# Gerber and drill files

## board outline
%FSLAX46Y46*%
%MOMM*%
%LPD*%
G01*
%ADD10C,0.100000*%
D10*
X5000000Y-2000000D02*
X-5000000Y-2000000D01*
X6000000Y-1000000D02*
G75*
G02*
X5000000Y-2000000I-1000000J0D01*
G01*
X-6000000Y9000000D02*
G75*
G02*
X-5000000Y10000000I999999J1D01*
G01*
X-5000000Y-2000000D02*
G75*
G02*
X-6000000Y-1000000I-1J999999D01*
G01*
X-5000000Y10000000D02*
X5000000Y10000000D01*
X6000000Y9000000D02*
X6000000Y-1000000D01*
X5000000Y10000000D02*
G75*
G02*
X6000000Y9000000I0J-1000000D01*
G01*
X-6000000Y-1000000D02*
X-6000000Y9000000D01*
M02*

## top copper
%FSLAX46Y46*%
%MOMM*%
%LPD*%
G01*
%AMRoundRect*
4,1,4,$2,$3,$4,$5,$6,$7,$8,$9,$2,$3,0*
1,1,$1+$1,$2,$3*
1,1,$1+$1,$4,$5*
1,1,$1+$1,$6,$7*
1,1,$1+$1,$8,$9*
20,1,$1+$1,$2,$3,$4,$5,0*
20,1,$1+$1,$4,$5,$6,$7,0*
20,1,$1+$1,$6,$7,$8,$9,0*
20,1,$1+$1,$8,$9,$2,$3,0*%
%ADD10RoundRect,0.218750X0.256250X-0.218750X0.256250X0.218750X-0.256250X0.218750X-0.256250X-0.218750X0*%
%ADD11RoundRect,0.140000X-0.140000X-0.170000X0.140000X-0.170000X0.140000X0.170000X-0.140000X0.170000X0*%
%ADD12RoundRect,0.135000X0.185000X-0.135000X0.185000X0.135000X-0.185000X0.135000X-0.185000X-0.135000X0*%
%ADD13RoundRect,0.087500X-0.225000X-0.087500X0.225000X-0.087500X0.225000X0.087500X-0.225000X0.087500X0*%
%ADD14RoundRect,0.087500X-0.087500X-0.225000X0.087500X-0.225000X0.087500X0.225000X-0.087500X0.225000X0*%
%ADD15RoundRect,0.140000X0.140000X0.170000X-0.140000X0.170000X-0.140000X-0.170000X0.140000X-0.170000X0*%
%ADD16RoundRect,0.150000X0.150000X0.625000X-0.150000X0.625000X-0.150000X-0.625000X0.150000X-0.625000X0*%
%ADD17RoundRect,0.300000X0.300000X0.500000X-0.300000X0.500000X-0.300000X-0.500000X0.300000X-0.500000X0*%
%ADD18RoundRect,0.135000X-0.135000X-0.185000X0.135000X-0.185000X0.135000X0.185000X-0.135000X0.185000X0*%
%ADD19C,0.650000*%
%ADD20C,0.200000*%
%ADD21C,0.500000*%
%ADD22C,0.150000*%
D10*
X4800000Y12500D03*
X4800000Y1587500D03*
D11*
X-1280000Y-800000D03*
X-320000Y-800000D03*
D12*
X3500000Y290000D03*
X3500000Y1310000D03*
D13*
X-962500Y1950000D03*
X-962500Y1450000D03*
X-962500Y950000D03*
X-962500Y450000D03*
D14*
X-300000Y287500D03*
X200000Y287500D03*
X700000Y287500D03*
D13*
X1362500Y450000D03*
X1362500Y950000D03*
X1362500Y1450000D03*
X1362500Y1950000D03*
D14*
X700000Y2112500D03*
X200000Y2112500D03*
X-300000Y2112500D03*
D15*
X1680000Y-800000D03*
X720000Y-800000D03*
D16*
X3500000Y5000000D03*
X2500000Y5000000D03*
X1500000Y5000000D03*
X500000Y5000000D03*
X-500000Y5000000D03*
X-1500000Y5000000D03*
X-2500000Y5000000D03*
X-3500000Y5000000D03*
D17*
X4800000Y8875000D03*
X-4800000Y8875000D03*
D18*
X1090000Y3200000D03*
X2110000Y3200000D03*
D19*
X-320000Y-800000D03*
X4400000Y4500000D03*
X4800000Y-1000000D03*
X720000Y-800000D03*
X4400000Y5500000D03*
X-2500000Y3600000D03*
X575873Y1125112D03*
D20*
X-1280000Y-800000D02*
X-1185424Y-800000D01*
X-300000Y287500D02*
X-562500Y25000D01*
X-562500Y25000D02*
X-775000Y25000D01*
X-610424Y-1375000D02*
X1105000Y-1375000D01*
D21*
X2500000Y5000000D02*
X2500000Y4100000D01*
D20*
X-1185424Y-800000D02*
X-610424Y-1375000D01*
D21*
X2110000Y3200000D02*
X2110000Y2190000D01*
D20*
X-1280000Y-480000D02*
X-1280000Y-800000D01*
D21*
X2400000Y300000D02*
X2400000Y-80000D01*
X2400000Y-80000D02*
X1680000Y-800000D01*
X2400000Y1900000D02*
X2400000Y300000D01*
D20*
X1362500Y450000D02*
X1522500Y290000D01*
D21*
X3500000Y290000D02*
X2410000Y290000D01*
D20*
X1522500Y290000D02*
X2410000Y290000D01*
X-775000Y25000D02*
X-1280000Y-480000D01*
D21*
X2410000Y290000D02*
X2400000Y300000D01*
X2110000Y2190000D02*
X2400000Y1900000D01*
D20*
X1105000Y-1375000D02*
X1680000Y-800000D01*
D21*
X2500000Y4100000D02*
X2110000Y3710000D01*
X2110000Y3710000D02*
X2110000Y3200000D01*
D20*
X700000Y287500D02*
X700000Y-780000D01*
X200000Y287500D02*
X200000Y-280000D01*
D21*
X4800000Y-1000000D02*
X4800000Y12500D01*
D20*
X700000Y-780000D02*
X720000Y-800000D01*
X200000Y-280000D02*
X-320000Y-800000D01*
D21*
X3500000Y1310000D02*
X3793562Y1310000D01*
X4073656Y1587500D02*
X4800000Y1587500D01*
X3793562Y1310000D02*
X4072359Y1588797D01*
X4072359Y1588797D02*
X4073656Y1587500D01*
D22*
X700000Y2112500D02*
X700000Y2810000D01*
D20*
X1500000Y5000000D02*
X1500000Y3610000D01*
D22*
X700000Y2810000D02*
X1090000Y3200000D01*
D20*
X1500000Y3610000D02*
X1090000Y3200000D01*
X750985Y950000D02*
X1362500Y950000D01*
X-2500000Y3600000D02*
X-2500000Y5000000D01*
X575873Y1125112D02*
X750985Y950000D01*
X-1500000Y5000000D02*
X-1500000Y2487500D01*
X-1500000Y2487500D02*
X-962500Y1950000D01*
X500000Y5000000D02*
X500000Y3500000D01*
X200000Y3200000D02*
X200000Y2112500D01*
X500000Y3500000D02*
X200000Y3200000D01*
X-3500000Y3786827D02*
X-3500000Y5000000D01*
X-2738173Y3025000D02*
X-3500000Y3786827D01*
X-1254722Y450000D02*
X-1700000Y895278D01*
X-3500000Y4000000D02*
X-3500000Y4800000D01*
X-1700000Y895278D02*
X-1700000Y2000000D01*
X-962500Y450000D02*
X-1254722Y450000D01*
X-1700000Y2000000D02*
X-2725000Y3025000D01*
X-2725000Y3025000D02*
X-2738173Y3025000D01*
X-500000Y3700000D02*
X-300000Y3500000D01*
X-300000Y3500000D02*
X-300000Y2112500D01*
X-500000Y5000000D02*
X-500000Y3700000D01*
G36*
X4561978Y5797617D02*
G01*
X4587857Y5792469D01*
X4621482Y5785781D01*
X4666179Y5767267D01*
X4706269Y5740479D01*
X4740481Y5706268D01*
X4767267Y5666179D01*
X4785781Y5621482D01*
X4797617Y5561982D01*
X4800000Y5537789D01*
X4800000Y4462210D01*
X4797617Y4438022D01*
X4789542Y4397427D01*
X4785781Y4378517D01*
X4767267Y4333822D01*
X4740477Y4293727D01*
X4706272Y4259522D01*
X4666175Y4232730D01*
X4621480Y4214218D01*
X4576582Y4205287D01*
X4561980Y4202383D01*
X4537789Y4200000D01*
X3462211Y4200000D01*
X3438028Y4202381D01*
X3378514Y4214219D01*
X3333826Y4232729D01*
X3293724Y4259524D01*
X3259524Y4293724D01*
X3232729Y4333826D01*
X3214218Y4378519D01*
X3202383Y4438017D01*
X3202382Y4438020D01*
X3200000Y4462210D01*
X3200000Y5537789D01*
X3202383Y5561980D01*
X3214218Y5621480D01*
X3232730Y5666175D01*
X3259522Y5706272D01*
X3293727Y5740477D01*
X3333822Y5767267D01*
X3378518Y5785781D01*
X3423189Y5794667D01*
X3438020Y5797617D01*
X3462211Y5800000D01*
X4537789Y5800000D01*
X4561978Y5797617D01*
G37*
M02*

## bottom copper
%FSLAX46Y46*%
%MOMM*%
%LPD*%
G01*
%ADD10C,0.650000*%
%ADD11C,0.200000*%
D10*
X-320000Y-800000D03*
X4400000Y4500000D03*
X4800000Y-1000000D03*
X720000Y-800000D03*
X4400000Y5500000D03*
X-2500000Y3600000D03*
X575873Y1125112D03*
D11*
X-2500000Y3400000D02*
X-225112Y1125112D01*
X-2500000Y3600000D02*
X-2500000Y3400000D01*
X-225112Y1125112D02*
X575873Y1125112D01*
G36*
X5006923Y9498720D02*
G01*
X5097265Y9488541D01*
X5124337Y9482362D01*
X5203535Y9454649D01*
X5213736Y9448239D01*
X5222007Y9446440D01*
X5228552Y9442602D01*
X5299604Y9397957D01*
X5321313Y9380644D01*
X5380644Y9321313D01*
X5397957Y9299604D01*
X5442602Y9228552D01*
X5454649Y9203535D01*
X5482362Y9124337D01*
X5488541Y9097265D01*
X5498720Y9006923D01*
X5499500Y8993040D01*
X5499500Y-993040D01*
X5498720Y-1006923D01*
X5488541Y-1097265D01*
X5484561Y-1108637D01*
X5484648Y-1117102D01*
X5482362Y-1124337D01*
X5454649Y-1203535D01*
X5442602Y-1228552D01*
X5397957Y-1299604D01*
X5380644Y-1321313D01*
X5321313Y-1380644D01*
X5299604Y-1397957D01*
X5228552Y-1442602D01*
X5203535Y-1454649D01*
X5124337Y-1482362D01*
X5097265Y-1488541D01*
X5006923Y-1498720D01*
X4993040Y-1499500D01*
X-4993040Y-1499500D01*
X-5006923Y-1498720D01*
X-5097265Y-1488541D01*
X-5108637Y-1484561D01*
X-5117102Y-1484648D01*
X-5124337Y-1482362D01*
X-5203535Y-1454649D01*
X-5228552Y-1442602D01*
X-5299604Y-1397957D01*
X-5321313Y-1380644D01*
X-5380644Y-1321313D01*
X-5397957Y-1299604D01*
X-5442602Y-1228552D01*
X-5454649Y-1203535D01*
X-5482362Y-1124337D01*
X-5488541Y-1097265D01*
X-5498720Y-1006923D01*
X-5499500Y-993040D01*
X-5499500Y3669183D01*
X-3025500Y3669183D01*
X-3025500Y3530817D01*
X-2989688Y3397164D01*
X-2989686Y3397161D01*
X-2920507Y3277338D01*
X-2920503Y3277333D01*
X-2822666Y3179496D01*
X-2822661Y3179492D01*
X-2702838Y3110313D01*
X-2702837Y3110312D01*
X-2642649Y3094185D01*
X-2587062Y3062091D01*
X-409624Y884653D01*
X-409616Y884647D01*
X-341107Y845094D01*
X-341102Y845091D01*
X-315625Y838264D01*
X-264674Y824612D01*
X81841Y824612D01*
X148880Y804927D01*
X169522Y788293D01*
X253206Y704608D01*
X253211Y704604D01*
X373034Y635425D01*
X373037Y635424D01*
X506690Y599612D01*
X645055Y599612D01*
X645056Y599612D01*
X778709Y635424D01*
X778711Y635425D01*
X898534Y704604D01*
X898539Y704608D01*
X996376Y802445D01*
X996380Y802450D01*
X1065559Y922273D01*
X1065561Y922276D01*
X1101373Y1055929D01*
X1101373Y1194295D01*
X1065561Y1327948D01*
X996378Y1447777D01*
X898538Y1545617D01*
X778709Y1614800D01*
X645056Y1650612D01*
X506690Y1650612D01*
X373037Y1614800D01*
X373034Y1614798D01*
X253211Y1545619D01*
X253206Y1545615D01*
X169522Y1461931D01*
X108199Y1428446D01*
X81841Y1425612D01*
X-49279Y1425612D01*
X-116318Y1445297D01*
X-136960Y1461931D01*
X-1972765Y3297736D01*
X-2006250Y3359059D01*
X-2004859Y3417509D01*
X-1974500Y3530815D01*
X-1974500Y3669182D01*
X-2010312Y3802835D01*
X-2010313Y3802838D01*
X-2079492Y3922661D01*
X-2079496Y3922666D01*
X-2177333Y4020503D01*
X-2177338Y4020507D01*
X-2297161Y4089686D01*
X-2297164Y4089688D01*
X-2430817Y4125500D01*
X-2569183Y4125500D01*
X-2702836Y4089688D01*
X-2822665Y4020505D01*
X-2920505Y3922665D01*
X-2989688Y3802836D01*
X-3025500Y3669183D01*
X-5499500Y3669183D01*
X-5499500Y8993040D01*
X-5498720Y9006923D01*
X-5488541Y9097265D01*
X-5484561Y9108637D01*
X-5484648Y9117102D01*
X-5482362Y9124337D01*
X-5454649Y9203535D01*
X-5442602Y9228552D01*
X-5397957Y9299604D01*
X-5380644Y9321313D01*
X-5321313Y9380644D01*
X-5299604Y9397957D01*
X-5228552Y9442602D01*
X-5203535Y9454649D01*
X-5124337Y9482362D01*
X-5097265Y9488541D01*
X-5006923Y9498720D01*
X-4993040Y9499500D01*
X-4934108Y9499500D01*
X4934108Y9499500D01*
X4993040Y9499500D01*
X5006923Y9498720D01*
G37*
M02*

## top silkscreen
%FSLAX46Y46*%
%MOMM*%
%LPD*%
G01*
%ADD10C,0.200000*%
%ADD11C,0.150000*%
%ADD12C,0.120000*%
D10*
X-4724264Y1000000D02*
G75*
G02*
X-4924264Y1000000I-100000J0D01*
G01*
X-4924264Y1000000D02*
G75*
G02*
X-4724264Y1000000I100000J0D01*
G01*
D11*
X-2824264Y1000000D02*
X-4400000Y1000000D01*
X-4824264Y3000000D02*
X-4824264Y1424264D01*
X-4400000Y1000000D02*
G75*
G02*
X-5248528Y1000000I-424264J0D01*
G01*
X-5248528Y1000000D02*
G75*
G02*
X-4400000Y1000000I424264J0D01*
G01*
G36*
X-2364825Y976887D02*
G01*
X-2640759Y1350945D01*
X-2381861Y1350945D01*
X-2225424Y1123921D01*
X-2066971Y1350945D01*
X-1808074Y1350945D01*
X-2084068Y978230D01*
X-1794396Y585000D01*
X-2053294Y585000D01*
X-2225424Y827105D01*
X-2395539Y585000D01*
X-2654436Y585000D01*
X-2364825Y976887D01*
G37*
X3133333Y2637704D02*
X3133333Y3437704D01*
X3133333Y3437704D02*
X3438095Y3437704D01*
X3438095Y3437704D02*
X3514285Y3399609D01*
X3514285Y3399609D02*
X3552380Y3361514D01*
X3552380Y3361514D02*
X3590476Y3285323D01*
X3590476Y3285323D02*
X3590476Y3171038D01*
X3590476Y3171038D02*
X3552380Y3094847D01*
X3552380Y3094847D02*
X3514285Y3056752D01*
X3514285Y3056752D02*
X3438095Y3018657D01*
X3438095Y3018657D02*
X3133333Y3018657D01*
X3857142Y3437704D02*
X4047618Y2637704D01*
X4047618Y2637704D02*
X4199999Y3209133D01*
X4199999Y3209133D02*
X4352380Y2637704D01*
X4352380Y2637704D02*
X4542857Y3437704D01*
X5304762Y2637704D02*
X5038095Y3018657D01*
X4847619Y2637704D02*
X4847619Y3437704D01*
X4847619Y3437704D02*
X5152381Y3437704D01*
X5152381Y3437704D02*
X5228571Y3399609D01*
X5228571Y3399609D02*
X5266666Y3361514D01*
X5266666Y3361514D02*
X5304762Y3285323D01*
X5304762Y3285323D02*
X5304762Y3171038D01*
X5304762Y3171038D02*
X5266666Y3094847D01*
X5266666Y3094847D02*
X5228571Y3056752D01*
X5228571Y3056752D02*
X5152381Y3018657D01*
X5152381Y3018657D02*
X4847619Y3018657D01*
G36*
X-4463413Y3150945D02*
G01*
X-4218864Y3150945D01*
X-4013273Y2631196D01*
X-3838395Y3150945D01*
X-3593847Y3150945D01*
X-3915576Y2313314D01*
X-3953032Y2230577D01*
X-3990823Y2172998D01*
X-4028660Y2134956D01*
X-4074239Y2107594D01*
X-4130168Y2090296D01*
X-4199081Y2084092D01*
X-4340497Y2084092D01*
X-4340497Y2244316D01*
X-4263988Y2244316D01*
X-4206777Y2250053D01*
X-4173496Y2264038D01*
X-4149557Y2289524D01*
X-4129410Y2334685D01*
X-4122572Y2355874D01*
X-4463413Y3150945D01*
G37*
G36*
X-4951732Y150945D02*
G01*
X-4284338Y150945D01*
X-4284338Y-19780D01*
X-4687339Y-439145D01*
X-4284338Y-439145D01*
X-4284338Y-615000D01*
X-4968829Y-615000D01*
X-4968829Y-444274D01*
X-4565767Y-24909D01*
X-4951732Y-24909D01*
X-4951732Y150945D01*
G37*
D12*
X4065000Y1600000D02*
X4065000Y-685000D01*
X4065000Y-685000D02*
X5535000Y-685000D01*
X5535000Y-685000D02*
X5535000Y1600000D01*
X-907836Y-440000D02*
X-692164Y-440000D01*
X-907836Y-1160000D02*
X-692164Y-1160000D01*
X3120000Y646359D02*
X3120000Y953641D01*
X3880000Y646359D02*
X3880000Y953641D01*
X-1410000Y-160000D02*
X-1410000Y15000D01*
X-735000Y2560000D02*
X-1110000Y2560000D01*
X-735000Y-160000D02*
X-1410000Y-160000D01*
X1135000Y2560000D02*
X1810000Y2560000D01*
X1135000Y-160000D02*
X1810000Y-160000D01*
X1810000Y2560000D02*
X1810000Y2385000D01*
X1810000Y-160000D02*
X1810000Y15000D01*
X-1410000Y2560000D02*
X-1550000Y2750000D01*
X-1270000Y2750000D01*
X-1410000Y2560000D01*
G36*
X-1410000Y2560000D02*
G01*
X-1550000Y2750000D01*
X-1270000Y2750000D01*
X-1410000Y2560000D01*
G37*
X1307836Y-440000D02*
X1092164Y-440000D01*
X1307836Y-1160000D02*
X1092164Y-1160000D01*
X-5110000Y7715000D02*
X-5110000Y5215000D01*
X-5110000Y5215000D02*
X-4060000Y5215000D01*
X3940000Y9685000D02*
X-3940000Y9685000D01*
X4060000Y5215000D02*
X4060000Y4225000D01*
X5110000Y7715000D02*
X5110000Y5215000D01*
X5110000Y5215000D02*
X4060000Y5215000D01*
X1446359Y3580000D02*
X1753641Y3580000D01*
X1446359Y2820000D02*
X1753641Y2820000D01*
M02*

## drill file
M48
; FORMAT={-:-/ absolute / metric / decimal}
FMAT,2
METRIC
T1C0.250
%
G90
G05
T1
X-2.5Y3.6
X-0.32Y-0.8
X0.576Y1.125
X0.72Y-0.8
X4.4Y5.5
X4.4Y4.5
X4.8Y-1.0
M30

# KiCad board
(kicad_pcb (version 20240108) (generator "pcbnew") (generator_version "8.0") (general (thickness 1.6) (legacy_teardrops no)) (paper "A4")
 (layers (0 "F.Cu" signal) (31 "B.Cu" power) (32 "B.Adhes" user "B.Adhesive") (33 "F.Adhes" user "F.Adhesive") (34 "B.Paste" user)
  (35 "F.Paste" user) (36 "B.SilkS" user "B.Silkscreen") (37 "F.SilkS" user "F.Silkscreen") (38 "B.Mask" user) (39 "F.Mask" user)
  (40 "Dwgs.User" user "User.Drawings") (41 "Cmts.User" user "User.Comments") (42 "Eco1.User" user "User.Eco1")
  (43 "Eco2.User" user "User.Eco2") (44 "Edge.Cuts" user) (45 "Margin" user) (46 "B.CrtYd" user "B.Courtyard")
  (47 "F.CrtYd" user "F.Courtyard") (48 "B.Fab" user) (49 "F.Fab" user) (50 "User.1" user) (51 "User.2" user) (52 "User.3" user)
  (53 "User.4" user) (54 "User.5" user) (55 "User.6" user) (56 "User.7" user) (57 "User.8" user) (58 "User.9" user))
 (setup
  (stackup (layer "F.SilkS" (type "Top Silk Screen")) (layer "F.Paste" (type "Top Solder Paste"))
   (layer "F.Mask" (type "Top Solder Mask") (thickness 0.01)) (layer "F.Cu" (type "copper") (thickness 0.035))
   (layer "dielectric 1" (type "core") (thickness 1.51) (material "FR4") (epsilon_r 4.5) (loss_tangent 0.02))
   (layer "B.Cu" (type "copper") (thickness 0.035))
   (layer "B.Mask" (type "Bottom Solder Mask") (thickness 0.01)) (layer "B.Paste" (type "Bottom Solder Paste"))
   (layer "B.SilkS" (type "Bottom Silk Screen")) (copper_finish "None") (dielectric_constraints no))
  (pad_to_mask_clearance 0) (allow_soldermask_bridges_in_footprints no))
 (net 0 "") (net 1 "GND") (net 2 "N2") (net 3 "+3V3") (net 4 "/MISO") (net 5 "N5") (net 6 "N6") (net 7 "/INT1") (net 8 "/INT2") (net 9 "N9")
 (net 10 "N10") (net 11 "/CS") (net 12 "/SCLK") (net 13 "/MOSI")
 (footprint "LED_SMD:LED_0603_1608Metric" (layer "F.Cu") (at 4.8 -0.8 90)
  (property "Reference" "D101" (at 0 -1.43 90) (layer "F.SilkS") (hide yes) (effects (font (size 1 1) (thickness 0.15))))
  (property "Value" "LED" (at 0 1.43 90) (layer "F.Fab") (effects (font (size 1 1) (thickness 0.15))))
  (fp_line (start 0.8 -0.735) (end -1.485 -0.735) (stroke (width 0.12) (type solid)) (layer "F.SilkS"))
  (fp_line (start -1.485 -0.735) (end -1.485 0.735) (stroke (width 0.12) (type solid)) (layer "F.SilkS"))
  (fp_line (start -1.485 0.735) (end 0.8 0.735) (stroke (width 0.12) (type solid)) (layer "F.SilkS"))
  (pad "1" smd roundrect (at -0.7875 0 90) (size 0.875 0.95) (layers "F.Cu" "F.Paste" "F.Mask") (roundrect_rratio 0.25) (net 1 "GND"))
  (pad "2" smd roundrect (at 0.7875 0 90) (size 0.875 0.95) (layers "F.Cu" "F.Paste" "F.Mask") (roundrect_rratio 0.25) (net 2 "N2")))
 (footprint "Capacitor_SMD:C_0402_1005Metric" (layer "F.Cu") (at -0.8 0.8)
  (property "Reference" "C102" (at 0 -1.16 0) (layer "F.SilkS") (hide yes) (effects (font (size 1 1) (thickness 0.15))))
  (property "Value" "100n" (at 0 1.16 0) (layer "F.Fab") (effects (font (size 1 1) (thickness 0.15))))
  (fp_line (start -0.107836 -0.36) (end 0.107836 -0.36) (stroke (width 0.12) (type solid)) (layer "F.SilkS"))
  (fp_line (start -0.107836 0.36) (end 0.107836 0.36) (stroke (width 0.12) (type solid)) (layer "F.SilkS"))
  (pad "1" smd roundrect (at -0.48 0) (size 0.56 0.62) (layers "F.Cu" "F.Paste" "F.Mask") (roundrect_rratio 0.25) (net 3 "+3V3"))
  (pad "2" smd roundrect (at 0.48 0) (size 0.56 0.62) (layers "F.Cu" "F.Paste" "F.Mask") (roundrect_rratio 0.25) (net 1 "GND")))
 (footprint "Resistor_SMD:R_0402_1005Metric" (layer "F.Cu") (at 3.5 -0.8 90)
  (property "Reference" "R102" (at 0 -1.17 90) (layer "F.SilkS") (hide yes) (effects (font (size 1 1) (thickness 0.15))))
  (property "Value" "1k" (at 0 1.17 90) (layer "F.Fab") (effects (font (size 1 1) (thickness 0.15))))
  (fp_line (start -0.153641 -0.38) (end 0.153641 -0.38) (stroke (width 0.12) (type solid)) (layer "F.SilkS"))
  (fp_line (start -0.153641 0.38) (end 0.153641 0.38) (stroke (width 0.12) (type solid)) (layer "F.SilkS"))
  (pad "1" smd roundrect (at -0.51 0 90) (size 0.54 0.64) (layers "F.Cu" "F.Paste" "F.Mask") (roundrect_rratio 0.25) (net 3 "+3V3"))
  (pad "2" smd roundrect (at 0.51 0 90) (size 0.54 0.64) (layers "F.Cu" "F.Paste" "F.Mask") (roundrect_rratio 0.25) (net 2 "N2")))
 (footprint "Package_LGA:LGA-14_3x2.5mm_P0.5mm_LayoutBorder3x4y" (layer "F.Cu") (at 0.2 -1.2)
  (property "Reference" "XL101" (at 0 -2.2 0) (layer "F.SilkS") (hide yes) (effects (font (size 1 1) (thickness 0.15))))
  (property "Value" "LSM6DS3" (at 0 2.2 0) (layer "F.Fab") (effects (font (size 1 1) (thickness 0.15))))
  (fp_line (start -1.61 1.36) (end -1.61 1.185) (stroke (width 0.12) (type solid)) (layer "F.SilkS"))
  (fp_line (start -0.935 -1.36) (end -1.31 -1.36) (stroke (width 0.12) (type solid)) (layer "F.SilkS"))
  (fp_line (start -0.935 1.36) (end -1.61 1.36) (stroke (width 0.12) (type solid)) (layer "F.SilkS"))
  (fp_line (start 0.935 -1.36) (end 1.61 -1.36) (stroke (width 0.12) (type solid)) (layer "F.SilkS"))
  (fp_line (start 0.935 1.36) (end 1.61 1.36) (stroke (width 0.12) (type solid)) (layer "F.SilkS"))
  (fp_line (start 1.61 -1.36) (end 1.61 -1.185) (stroke (width 0.12) (type solid)) (layer "F.SilkS"))
  (fp_line (start 1.61 1.36) (end 1.61 1.185) (stroke (width 0.12) (type solid)) (layer "F.SilkS"))
  (fp_poly
   (pts (xy -1.61 -1.36) (xy -1.75 -1.55) (xy -1.47 -1.55) (xy -1.61 -1.36)) (stroke (width 0.12) (type solid)) (fill solid)
   (layer "F.SilkS"))
  (pad "1" smd roundrect (at -1.1625 -0.75) (size 0.625 0.35) (layers "F.Cu" "F.Paste" "F.Mask") (roundrect_rratio 0.25) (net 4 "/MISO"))
  (pad "2" smd roundrect (at -1.1625 -0.25) (size 0.625 0.35) (layers "F.Cu" "F.Paste" "F.Mask") (roundrect_rratio 0.25) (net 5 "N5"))
  (pad "3" smd roundrect (at -1.1625 0.25) (size 0.625 0.35) (layers "F.Cu" "F.Paste" "F.Mask") (roundrect_rratio 0.25) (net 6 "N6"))
  (pad "4" smd roundrect (at -1.1625 0.75) (size 0.625 0.35) (layers "F.Cu" "F.Paste" "F.Mask") (roundrect_rratio 0.25) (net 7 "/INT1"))
  (pad "5" smd roundrect (at -0.5 0.9125) (size 0.35 0.625) (layers "F.Cu" "F.Paste" "F.Mask") (roundrect_rratio 0.25) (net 3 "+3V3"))
  (pad "6" smd roundrect (at 0 0.9125) (size 0.35 0.625) (layers "F.Cu" "F.Paste" "F.Mask") (roundrect_rratio 0.25) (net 1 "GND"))
  (pad "7" smd roundrect (at 0.5 0.9125) (size 0.35 0.625) (layers "F.Cu" "F.Paste" "F.Mask") (roundrect_rratio 0.25) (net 1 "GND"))
  (pad "8" smd roundrect (at 1.1625 0.75) (size 0.625 0.35) (layers "F.Cu" "F.Paste" "F.Mask") (roundrect_rratio 0.25) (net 3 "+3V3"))
  (pad "9" smd roundrect (at 1.1625 0.25) (size 0.625 0.35) (layers "F.Cu" "F.Paste" "F.Mask") (roundrect_rratio 0.25) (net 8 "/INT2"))
  (pad "10" smd roundrect (at 1.1625 -0.25) (size 0.625 0.35) (layers "F.Cu" "F.Paste" "F.Mask") (roundrect_rratio 0.25) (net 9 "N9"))
  (pad "11" smd roundrect (at 1.1625 -0.75) (size 0.625 0.35) (layers "F.Cu" "F.Paste" "F.Mask") (roundrect_rratio 0.25) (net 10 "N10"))
  (pad "12" smd roundrect (at 0.5 -0.9125) (size 0.35 0.625) (layers "F.Cu" "F.Paste" "F.Mask") (roundrect_rratio 0.25) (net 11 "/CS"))
  (pad "13" smd roundrect (at 0 -0.9125) (size 0.35 0.625) (layers "F.Cu" "F.Paste" "F.Mask") (roundrect_rratio 0.25) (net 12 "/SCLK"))
  (pad "14" smd roundrect (at -0.5 -0.9125) (size 0.35 0.625) (layers "F.Cu" "F.Paste" "F.Mask") (roundrect_rratio 0.25) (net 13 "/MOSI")))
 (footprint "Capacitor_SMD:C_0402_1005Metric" (layer "F.Cu") (at 1.2 0.8 180)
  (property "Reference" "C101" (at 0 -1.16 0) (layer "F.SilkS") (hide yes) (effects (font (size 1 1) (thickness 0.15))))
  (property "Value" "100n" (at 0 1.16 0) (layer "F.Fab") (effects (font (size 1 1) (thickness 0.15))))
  (fp_line (start -0.107836 0.36) (end 0.107836 0.36) (stroke (width 0.12) (type solid)) (layer "F.SilkS"))
  (fp_line (start -0.107836 -0.36) (end 0.107836 -0.36) (stroke (width 0.12) (type solid)) (layer "F.SilkS"))
  (pad "1" smd roundrect (at -0.48 0 180) (size 0.56 0.62) (layers "F.Cu" "F.Paste" "F.Mask") (roundrect_rratio 0.25) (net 3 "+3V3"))
  (pad "2" smd roundrect (at 0.48 0 180) (size 0.56 0.62) (layers "F.Cu" "F.Paste" "F.Mask") (roundrect_rratio 0.25) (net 1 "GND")))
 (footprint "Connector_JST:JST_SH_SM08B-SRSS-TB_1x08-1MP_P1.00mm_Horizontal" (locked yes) (layer "F.Cu") (at 0 -7 180)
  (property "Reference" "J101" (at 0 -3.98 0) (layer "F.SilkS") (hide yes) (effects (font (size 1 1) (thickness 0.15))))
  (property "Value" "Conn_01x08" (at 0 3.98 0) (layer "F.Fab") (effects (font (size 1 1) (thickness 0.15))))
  (fp_line (start 5.11 0.715) (end 5.11 -1.785) (stroke (width 0.12) (type solid)) (layer "F.SilkS"))
  (fp_line (start 5.11 -1.785) (end 4.06 -1.785) (stroke (width 0.12) (type solid)) (layer "F.SilkS"))
  (fp_line (start -3.94 2.685) (end 3.94 2.685) (stroke (width 0.12) (type solid)) (layer "F.SilkS"))
  (fp_line (start -4.06 -1.785) (end -4.06 -2.775) (stroke (width 0.12) (type solid)) (layer "F.SilkS"))
  (fp_line (start -5.11 0.715) (end -5.11 -1.785) (stroke (width 0.12) (type solid)) (layer "F.SilkS"))
  (fp_line (start -5.11 -1.785) (end -4.06 -1.785) (stroke (width 0.12) (type solid)) (layer "F.SilkS"))
  (pad "1" smd roundrect (at -3.5 -2 180) (size 0.6 1.55) (layers "F.Cu" "F.Paste" "F.Mask") (roundrect_rratio 0.25) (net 1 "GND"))
  (pad "2" smd roundrect (at -2.5 -2 180) (size 0.6 1.55) (layers "F.Cu" "F.Paste" "F.Mask") (roundrect_rratio 0.25) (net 3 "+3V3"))
  (pad "3" smd roundrect (at -1.5 -2 180) (size 0.6 1.55) (layers "F.Cu" "F.Paste" "F.Mask") (roundrect_rratio 0.25) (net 11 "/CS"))
  (pad "4" smd roundrect (at -0.5 -2 180) (size 0.6 1.55) (layers "F.Cu" "F.Paste" "F.Mask") (roundrect_rratio 0.25) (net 12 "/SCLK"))
  (pad "5" smd roundrect (at 0.5 -2 180) (size 0.6 1.55) (layers "F.Cu" "F.Paste" "F.Mask") (roundrect_rratio 0.25) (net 13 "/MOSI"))
  (pad "6" smd roundrect (at 1.5 -2 180) (size 0.6 1.55) (layers "F.Cu" "F.Paste" "F.Mask") (roundrect_rratio 0.25) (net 4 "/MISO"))
  (pad "7" smd roundrect (at 2.5 -2 180) (size 0.6 1.55) (layers "F.Cu" "F.Paste" "F.Mask") (roundrect_rratio 0.25) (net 8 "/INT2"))
  (pad "8" smd roundrect (at 3.5 -2 180) (size 0.6 1.55) (layers "F.Cu" "F.Paste" "F.Mask") (roundrect_rratio 0.25) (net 7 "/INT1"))
  (pad "MP" smd roundrect (at -4.8 1.875 180) (size 1.2 1.6) (layers "F.Cu" "F.Paste" "F.Mask") (roundrect_rratio 0.25))
  (pad "MP" smd roundrect (at 4.8 1.875 180) (size 1.2 1.6) (layers "F.Cu" "F.Paste" "F.Mask") (roundrect_rratio 0.25)))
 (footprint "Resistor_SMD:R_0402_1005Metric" (layer "F.Cu") (at 1.6 -3.2)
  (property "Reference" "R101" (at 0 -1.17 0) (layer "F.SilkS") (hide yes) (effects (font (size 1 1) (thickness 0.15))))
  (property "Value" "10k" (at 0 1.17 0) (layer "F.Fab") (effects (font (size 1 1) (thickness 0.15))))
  (fp_line (start -0.153641 -0.38) (end 0.153641 -0.38) (stroke (width 0.12) (type solid)) (layer "F.SilkS"))
  (fp_line (start -0.153641 0.38) (end 0.153641 0.38) (stroke (width 0.12) (type solid)) (layer "F.SilkS"))
  (pad "1" smd roundrect (at -0.51 0) (size 0.54 0.64) (layers "F.Cu" "F.Paste" "F.Mask") (roundrect_rratio 0.25) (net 11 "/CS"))
  (pad "2" smd roundrect (at 0.51 0) (size 0.54 0.64) (layers "F.Cu" "F.Paste" "F.Mask") (roundrect_rratio 0.25) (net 3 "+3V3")))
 (gr_circle (center -4.824264 -1) (end -4.824264 -0.9) (stroke (width 0.2) (type default)) (fill none) (layer "F.SilkS"))
 (gr_line (start -2.824264 -1) (end -4.4 -1) (stroke (width 0.15) (type default)) (layer "F.SilkS"))
 (gr_line (start -4.824264 -3) (end -4.824264 -1.424264) (stroke (width 0.15) (type default)) (layer "F.SilkS"))
 (gr_circle (center -4.824264 -1) (end -4.524264 -1.3) (stroke (width 0.15) (type default)) (fill none) (layer "F.SilkS"))
 (gr_line (start 5 2) (end -5 2) (stroke (width 0.1) (type default)) (layer "Edge.Cuts"))
 (gr_arc (start 6 1) (mid 5.707107 1.707107) (end 5 2) (stroke (width 0.1) (type default)) (layer "Edge.Cuts"))
 (gr_arc (start -6 -9) (mid -5.707107 -9.707107) (end -5 -10) (stroke (width 0.1) (type default)) (layer "Edge.Cuts"))
 (gr_arc (start -5 2) (mid -5.707107 1.707107) (end -6 1) (stroke (width 0.1) (type default)) (layer "Edge.Cuts"))
 (gr_line (start -5 -10) (end 5 -10) (stroke (width 0.1) (type default)) (layer "Edge.Cuts"))
 (gr_line (start 6 -9) (end 6 1) (stroke (width 0.1) (type default)) (layer "Edge.Cuts"))
 (gr_arc (start 5 -10) (mid 5.707107 -9.707107) (end 6 -9) (stroke (width 0.1) (type default)) (layer "Edge.Cuts"))
 (gr_line (start -6 1) (end -6 -9) (stroke (width 0.1) (type default)) (layer "Edge.Cuts"))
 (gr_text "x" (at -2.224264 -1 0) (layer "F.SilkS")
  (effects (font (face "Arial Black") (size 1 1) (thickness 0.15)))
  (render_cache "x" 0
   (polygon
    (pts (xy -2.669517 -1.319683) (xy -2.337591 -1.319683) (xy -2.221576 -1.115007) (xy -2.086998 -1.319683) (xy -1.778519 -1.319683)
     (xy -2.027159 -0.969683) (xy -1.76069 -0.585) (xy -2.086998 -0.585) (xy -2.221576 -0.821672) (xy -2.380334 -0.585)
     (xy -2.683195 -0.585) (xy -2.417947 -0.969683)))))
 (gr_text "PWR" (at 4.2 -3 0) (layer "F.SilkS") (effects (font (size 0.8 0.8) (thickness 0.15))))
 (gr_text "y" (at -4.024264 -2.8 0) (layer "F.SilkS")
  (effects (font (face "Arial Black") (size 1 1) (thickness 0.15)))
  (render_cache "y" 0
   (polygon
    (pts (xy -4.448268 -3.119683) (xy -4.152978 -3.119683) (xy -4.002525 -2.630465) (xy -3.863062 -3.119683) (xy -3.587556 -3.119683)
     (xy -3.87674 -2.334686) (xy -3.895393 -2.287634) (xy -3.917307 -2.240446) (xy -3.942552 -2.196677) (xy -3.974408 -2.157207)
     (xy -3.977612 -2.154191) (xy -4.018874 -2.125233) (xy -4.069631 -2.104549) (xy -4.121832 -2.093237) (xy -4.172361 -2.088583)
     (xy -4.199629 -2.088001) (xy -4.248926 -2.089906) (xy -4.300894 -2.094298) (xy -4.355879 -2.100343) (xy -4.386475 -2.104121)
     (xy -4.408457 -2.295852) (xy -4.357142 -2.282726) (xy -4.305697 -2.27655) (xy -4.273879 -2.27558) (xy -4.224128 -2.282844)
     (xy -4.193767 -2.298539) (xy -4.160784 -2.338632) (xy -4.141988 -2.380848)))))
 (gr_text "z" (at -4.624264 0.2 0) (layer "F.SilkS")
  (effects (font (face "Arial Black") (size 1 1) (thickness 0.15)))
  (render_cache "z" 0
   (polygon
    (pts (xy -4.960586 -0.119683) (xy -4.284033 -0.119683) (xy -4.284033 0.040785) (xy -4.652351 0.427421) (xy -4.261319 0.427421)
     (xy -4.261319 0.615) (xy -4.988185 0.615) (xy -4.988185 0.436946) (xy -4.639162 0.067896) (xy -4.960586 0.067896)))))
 (segment (start -1.28 0.8) (end -1.185424 0.8) (width 0.2) (layer "F.Cu") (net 3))
 (segment (start -0.3 -0.2875) (end -0.5625 -0.025) (width 0.2) (layer "F.Cu") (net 3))
 (segment (start -0.5625 -0.025) (end -0.775 -0.025) (width 0.2) (layer "F.Cu") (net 3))
 (segment (start -0.610424 1.375) (end 1.105 1.375) (width 0.2) (layer "F.Cu") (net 3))
 (segment (start 2.5 -5) (end 2.5 -4.1) (width 0.5) (layer "F.Cu") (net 3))
 (segment (start -1.185424 0.8) (end -0.610424 1.375) (width 0.2) (layer "F.Cu") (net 3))
 (segment (start 2.11 -3.2) (end 2.11 -2.19) (width 0.5) (layer "F.Cu") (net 3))
 (segment (start -1.28 0.48) (end -1.28 0.8) (width 0.2) (layer "F.Cu") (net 3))
 (segment (start 2.4 -0.3) (end 2.4 0.08) (width 0.5) (layer "F.Cu") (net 3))
 (segment (start 2.4 0.08) (end 1.68 0.8) (width 0.5) (layer "F.Cu") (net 3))
 (segment (start 2.4 -1.9) (end 2.4 -0.3) (width 0.5) (layer "F.Cu") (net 3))
 (segment (start 1.3625 -0.45) (end 1.5225 -0.29) (width 0.2) (layer "F.Cu") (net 3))
 (segment (start 3.5 -0.29) (end 2.41 -0.29) (width 0.5) (layer "F.Cu") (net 3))
 (segment (start 1.5225 -0.29) (end 2.41 -0.29) (width 0.2) (layer "F.Cu") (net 3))
 (segment (start -0.775 -0.025) (end -1.28 0.48) (width 0.2) (layer "F.Cu") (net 3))
 (segment (start 2.41 -0.29) (end 2.4 -0.3) (width 0.5) (layer "F.Cu") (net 3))
 (segment (start 2.11 -2.19) (end 2.4 -1.9) (width 0.5) (layer "F.Cu") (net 3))
 (segment (start 1.105 1.375) (end 1.68 0.8) (width 0.2) (layer "F.Cu") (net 3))
 (segment (start 2.5 -4.1) (end 2.11 -3.71) (width 0.5) (layer "F.Cu") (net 3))
 (segment (start 2.11 -3.71) (end 2.11 -3.2) (width 0.5) (layer "F.Cu") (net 3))
 (segment (start 0.7 -0.2875) (end 0.7 0.78) (width 0.2) (layer "F.Cu") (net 1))
 (segment (start 0.2 -0.2875) (end 0.2 0.28) (width 0.2) (layer "F.Cu") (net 1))
 (segment (start 4.8 1) (end 4.8 -0.0125) (width 0.5) (layer "F.Cu") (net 1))
 (segment (start 0.7 0.78) (end 0.72 0.8) (width 0.2) (layer "F.Cu") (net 1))
 (segment (start 0.2 0.28) (end -0.32 0.8) (width 0.2) (layer "F.Cu") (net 1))
 (via (at -0.32 0.8) (size 0.65) (drill 0.25) (layers "F.Cu" "B.Cu") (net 1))
 (via (at 4.4 -4.5) (size 0.65) (drill 0.25) (layers "F.Cu" "B.Cu") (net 1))
 (via (at 4.8 1) (size 0.65) (drill 0.25) (layers "F.Cu" "B.Cu") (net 1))
 (via (at 0.72 0.8) (size 0.65) (drill 0.25) (layers "F.Cu" "B.Cu") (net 1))
 (via (at 4.4 -5.5) (size 0.65) (drill 0.25) (layers "F.Cu" "B.Cu") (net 1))
 (segment (start 3.5 -1.31) (end 3.793562 -1.31) (width 0.5) (layer "F.Cu") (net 2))
 (segment (start 4.073656 -1.5875) (end 4.8 -1.5875) (width 0.5) (layer "F.Cu") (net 2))
 (segment (start 3.793562 -1.31) (end 4.072359 -1.588797) (width 0.5) (layer "F.Cu") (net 2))
 (segment (start 4.072359 -1.588797) (end 4.073656 -1.5875) (width 0.5) (layer "F.Cu") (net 2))
 (segment (start 0.7 -2.1125) (end 0.7 -2.81) (width 0.15) (layer "F.Cu") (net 11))
 (segment (start 1.5 -5) (end 1.5 -3.61) (width 0.2) (layer "F.Cu") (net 11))
 (segment (start 0.7 -2.81) (end 1.09 -3.2) (width 0.15) (layer "F.Cu") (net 11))
 (segment (start 1.5 -3.61) (end 1.09 -3.2) (width 0.2) (layer "F.Cu") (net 11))
 (segment (start 0.750985 -0.95) (end 1.3625 -0.95) (width 0.2) (layer "F.Cu") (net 8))
 (segment (start -2.5 -3.6) (end -2.5 -5) (width 0.2) (layer "F.Cu") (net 8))
 (segment (start 0.575873 -1.125112) (end 0.750985 -0.95) (width 0.2) (layer "F.Cu") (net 8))
 (via (at -2.5 -3.6) (size 0.65) (drill 0.25) (layers "F.Cu" "B.Cu") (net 8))
 (via (at 0.575873 -1.125112) (size 0.65) (drill 0.25) (layers "F.Cu" "B.Cu") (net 8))
 (segment (start -2.5 -3.4) (end -0.225112 -1.125112) (width 0.2) (layer "B.Cu") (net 8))
 (segment (start -2.5 -3.6) (end -2.5 -3.4) (width 0.2) (layer "B.Cu") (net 8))
 (segment (start -0.225112 -1.125112) (end 0.575873 -1.125112) (width 0.2) (layer "B.Cu") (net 8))
 (segment (start -1.5 -5) (end -1.5 -2.4875) (width 0.2) (layer "F.Cu") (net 4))
 (segment (start -1.5 -2.4875) (end -0.9625 -1.95) (width 0.2) (layer "F.Cu") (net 4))
 (segment (start 0.5 -5) (end 0.5 -3.5) (width 0.2) (layer "F.Cu") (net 12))
 (segment (start 0.2 -3.2) (end 0.2 -2.1125) (width 0.2) (layer "F.Cu") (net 12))
 (segment (start 0.5 -3.5) (end 0.2 -3.2) (width 0.2) (layer "F.Cu") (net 12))
 (segment (start -3.5 -3.786827) (end -3.5 -5) (width 0.2) (layer "F.Cu") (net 7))
 (segment (start -2.738173 -3.025) (end -3.5 -3.786827) (width 0.2) (layer "F.Cu") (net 7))
 (segment (start -1.254722 -0.45) (end -1.7 -0.895278) (width 0.2) (layer "F.Cu") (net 7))
 (segment (start -3.5 -4) (end -3.5 -4.8) (width 0.2) (layer "F.Cu") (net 7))
 (segment (start -1.7 -0.895278) (end -1.7 -2) (width 0.2) (layer "F.Cu") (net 7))
 (segment (start -0.9625 -0.45) (end -1.254722 -0.45) (width 0.2) (layer "F.Cu") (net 7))
 (segment (start -1.7 -2) (end -2.725 -3.025) (width 0.2) (layer "F.Cu") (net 7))
 (segment (start -2.725 -3.025) (end -2.738173 -3.025) (width 0.2) (layer "F.Cu") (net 7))
 (segment (start -0.5 -3.7) (end -0.3 -3.5) (width 0.2) (layer "F.Cu") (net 13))
 (segment (start -0.3 -3.5) (end -0.3 -2.1125) (width 0.2) (layer "F.Cu") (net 13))
 (segment (start -0.5 -5) (end -0.5 -3.7) (width 0.2) (layer "F.Cu") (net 13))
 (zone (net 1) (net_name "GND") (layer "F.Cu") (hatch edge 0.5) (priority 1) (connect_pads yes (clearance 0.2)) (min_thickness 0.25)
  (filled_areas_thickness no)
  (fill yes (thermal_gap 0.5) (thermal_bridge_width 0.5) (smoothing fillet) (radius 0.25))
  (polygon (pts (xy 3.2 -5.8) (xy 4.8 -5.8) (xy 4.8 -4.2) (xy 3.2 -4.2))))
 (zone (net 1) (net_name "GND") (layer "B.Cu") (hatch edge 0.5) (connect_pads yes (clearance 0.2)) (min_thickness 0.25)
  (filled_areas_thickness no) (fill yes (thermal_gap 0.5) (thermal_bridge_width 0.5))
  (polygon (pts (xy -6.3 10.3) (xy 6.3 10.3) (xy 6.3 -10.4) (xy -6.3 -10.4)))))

